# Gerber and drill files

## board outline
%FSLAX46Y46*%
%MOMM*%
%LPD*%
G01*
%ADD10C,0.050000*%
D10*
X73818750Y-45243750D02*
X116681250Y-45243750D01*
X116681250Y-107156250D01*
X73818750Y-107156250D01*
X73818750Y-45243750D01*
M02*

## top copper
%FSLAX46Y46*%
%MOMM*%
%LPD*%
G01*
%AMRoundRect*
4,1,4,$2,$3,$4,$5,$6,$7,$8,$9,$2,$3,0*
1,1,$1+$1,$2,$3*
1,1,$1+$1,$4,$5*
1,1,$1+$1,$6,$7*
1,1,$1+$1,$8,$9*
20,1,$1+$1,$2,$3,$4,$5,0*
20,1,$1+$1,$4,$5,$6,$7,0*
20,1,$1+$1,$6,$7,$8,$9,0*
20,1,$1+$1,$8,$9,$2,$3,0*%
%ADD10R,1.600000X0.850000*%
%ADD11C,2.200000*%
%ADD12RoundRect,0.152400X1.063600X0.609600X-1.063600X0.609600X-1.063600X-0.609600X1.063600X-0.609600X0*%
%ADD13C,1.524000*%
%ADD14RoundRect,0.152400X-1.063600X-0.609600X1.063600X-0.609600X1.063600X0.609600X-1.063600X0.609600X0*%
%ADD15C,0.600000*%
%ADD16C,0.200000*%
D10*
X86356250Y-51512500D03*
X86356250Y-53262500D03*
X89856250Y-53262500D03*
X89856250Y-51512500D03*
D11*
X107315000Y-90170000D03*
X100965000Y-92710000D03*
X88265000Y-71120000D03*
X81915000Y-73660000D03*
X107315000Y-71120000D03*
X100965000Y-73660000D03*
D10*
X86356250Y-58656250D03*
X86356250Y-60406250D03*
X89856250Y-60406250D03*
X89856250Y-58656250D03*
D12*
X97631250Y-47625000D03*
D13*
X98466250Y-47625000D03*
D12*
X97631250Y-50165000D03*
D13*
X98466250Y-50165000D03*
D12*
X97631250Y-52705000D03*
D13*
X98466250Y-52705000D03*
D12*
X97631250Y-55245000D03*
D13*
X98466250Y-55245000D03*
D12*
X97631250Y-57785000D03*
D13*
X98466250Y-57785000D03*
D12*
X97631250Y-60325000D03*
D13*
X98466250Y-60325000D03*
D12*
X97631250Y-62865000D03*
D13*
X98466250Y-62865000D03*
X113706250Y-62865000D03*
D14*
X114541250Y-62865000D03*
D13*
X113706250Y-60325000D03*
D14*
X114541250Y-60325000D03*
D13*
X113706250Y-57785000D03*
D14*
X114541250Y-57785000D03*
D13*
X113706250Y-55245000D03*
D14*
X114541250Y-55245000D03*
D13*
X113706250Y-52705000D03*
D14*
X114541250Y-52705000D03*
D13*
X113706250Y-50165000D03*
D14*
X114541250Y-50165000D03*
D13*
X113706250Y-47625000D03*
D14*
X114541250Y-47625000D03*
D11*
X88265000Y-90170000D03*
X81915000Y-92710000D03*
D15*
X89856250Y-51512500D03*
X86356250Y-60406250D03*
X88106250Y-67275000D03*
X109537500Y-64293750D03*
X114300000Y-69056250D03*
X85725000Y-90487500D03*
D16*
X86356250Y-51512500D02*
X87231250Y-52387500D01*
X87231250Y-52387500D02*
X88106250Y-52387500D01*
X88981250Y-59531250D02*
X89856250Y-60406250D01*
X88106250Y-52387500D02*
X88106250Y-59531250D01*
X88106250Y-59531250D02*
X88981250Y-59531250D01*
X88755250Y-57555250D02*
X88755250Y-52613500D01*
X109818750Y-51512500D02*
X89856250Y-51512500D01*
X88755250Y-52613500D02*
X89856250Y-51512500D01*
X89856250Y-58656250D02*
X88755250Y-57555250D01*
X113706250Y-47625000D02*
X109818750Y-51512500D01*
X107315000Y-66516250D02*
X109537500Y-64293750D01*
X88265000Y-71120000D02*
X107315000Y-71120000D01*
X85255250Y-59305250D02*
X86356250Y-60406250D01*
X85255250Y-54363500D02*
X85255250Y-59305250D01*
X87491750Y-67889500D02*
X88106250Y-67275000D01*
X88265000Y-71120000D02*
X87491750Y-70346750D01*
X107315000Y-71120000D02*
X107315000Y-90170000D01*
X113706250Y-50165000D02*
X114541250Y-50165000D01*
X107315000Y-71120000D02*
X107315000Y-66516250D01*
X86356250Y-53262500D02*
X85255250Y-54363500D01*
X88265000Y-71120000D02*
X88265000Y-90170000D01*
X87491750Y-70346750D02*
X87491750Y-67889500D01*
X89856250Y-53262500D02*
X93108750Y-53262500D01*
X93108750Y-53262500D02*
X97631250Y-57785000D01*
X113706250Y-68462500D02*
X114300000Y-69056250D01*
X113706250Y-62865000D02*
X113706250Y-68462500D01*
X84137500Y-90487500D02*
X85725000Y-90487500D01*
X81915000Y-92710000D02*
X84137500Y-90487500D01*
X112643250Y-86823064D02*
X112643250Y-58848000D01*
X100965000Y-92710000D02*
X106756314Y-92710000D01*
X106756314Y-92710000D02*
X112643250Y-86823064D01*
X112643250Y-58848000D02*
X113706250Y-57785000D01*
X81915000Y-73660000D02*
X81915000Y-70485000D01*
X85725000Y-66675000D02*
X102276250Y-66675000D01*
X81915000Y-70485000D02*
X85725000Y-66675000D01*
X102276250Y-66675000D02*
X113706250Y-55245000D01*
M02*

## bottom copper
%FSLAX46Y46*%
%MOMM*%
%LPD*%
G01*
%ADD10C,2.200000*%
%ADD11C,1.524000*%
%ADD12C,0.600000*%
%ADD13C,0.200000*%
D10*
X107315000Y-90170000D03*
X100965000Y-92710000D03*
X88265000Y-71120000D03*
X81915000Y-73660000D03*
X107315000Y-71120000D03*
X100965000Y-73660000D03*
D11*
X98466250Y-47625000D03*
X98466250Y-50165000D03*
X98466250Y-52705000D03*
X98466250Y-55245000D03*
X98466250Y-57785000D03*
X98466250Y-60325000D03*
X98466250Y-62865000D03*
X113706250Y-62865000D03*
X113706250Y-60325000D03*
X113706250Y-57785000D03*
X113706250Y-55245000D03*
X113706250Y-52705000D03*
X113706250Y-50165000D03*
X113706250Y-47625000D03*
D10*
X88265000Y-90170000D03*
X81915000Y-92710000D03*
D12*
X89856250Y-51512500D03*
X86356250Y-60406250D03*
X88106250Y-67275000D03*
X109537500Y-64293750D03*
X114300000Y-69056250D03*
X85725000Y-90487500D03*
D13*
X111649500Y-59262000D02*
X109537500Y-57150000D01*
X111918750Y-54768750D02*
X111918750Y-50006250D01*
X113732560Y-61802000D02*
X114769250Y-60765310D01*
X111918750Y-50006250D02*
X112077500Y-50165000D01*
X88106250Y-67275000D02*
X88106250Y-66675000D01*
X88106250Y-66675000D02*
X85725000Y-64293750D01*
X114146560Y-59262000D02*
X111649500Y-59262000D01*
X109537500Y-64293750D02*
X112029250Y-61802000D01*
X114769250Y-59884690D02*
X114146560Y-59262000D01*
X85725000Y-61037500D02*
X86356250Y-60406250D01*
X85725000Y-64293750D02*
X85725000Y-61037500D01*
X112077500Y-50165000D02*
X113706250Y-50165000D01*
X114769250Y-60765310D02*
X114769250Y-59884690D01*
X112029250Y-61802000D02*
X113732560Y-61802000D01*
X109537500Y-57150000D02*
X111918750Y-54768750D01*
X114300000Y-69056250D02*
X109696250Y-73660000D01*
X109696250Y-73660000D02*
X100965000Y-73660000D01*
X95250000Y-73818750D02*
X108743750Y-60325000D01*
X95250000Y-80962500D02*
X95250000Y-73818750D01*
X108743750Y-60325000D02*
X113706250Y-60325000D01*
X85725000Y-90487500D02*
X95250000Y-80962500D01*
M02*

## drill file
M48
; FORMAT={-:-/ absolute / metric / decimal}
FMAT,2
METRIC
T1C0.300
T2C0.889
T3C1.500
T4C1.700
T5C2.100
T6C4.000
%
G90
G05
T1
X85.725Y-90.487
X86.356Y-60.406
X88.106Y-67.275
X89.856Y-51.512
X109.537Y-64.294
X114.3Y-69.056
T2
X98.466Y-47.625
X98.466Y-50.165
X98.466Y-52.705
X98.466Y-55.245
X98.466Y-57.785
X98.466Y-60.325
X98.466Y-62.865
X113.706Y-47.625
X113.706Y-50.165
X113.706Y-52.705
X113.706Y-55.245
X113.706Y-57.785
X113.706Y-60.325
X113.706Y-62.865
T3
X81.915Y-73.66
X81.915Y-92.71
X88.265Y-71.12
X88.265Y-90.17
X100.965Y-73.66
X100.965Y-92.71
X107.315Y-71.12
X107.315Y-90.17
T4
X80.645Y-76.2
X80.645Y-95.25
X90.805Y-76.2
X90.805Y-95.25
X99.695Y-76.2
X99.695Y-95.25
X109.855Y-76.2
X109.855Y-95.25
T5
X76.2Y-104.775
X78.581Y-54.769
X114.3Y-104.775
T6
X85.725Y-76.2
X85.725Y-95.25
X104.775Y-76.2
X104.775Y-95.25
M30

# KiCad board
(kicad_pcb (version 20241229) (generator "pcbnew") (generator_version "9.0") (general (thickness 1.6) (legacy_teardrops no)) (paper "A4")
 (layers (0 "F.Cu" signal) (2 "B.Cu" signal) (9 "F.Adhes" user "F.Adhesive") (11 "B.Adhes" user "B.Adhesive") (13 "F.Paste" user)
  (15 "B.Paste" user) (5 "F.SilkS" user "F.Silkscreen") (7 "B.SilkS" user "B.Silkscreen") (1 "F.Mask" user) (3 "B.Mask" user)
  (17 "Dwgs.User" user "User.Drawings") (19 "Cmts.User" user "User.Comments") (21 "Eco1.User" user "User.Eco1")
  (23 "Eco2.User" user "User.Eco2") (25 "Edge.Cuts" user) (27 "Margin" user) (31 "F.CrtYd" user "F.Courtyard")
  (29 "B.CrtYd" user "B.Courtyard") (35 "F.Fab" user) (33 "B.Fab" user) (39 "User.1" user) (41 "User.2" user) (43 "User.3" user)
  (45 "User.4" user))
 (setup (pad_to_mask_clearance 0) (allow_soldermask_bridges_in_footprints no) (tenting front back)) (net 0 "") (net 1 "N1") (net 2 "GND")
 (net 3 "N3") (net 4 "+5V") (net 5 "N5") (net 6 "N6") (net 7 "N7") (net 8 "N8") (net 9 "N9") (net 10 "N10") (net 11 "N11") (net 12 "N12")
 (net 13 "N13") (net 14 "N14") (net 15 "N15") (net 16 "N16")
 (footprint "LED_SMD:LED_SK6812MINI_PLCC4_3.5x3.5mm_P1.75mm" (layer "F.Cu") (at 88.10625 52.3875)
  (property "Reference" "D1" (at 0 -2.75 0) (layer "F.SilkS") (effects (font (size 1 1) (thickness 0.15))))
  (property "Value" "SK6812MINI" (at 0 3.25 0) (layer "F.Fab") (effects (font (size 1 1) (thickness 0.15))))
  (pad "1" smd rect (at -1.75 -0.875) (size 1.6 0.85) (layers "F.Cu" "F.Mask" "F.Paste") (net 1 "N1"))
  (pad "2" smd rect (at -1.75 0.875) (size 1.6 0.85) (layers "F.Cu" "F.Mask" "F.Paste") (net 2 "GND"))
  (pad "3" smd rect (at 1.75 0.875) (size 1.6 0.85) (layers "F.Cu" "F.Mask" "F.Paste") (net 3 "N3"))
  (pad "4" smd rect (at 1.75 -0.875) (size 1.6 0.85) (layers "F.Cu" "F.Mask" "F.Paste") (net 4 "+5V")))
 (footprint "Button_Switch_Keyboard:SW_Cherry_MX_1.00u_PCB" (layer "F.Cu") (at 107.315 90.17)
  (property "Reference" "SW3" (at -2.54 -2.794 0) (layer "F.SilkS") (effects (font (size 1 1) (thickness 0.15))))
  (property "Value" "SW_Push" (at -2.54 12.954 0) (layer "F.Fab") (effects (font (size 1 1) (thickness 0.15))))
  (pad "" np_thru_hole circle (at -7.62 5.08) (size 1.7 1.7) (drill 1.7) (layers "*.Cu" "*.Mask"))
  (pad "" np_thru_hole circle (at -2.54 5.08) (size 4 4) (drill 4) (layers "*.Cu" "*.Mask"))
  (pad "" np_thru_hole circle (at 2.54 5.08) (size 1.7 1.7) (drill 1.7) (layers "*.Cu" "*.Mask"))
  (pad "1" thru_hole circle (at 0 0) (size 2.2 2.2) (drill 1.5) (layers "*.Cu" "*.Mask") (remove_unused_layers no) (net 2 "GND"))
  (pad "2" thru_hole circle (at -6.35 2.54) (size 2.2 2.2) (drill 1.5) (layers "*.Cu" "*.Mask") (remove_unused_layers no) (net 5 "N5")))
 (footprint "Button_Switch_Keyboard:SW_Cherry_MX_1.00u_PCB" (layer "F.Cu") (at 88.265 71.12)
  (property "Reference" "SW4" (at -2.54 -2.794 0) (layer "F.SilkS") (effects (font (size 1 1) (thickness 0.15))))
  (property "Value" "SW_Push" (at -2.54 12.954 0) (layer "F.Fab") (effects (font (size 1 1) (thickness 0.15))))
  (pad "" np_thru_hole circle (at -7.62 5.08) (size 1.7 1.7) (drill 1.7) (layers "*.Cu" "*.Mask"))
  (pad "" np_thru_hole circle (at -2.54 5.08) (size 4 4) (drill 4) (layers "*.Cu" "*.Mask"))
  (pad "" np_thru_hole circle (at 2.54 5.08) (size 1.7 1.7) (drill 1.7) (layers "*.Cu" "*.Mask"))
  (pad "1" thru_hole circle (at 0 0) (size 2.2 2.2) (drill 1.5) (layers "*.Cu" "*.Mask") (remove_unused_layers no) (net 2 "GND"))
  (pad "2" thru_hole circle (at -6.35 2.54) (size 2.2 2.2) (drill 1.5) (layers "*.Cu" "*.Mask") (remove_unused_layers no) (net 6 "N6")))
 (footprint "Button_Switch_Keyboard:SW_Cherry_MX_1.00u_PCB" (layer "F.Cu") (at 107.315 71.12)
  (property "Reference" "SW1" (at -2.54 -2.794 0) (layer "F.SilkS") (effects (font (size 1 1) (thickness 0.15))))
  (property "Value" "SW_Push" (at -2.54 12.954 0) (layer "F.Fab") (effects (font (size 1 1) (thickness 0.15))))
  (pad "" np_thru_hole circle (at -7.62 5.08) (size 1.7 1.7) (drill 1.7) (layers "*.Cu" "*.Mask"))
  (pad "" np_thru_hole circle (at -2.54 5.08) (size 4 4) (drill 4) (layers "*.Cu" "*.Mask"))
  (pad "" np_thru_hole circle (at 2.54 5.08) (size 1.7 1.7) (drill 1.7) (layers "*.Cu" "*.Mask"))
  (pad "1" thru_hole circle (at 0 0) (size 2.2 2.2) (drill 1.5) (layers "*.Cu" "*.Mask") (remove_unused_layers no) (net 2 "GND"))
  (pad "2" thru_hole circle (at -6.35 2.54) (size 2.2 2.2) (drill 1.5) (layers "*.Cu" "*.Mask") (remove_unused_layers no) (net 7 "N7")))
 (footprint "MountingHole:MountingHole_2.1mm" (layer "F.Cu") (at 76.2 104.775)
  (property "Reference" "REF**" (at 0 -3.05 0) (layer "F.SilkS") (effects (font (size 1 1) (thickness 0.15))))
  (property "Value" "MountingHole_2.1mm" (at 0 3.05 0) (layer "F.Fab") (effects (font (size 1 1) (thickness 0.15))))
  (pad "" np_thru_hole circle (at 0 0) (size 2.1 2.1) (drill 2.1) (layers "*.Cu" "*.Mask")))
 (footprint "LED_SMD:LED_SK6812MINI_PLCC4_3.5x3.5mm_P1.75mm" (layer "F.Cu") (at 88.10625 59.53125)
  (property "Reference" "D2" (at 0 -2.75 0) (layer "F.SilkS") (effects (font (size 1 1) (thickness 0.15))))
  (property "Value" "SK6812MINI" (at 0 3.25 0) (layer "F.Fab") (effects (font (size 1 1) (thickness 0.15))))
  (pad "1" smd rect (at -1.75 -0.875) (size 1.6 0.85) (layers "F.Cu" "F.Mask" "F.Paste") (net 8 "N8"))
  (pad "2" smd rect (at -1.75 0.875) (size 1.6 0.85) (layers "F.Cu" "F.Mask" "F.Paste") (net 2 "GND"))
  (pad "3" smd rect (at 1.75 0.875) (size 1.6 0.85) (layers "F.Cu" "F.Mask" "F.Paste") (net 1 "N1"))
  (pad "4" smd rect (at 1.75 -0.875) (size 1.6 0.85) (layers "F.Cu" "F.Mask" "F.Paste") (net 4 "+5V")))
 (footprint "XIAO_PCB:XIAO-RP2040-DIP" (layer "F.Cu") (at 106.08625 55.245)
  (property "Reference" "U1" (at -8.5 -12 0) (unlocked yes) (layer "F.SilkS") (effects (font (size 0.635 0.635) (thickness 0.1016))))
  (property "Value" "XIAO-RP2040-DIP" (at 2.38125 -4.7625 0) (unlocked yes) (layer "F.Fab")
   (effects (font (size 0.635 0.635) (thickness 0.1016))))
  (pad "1" smd roundrect (at -8.455 -7.62 180) (size 2.432 1.524) (layers "F.Cu" "F.Mask") (roundrect_rratio 0.1) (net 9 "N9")
   (thermal_bridge_angle 45))
  (pad "1" thru_hole circle (at -7.62 -7.62 180) (size 1.524 1.524) (drill 0.889) (layers "*.Cu" "*.Mask") (remove_unused_layers no)
   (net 9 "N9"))
  (pad "2" smd roundrect (at -8.455 -5.08 180) (size 2.432 1.524) (layers "F.Cu" "F.Mask") (roundrect_rratio 0.1) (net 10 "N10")
   (thermal_bridge_angle 45))
  (pad "2" thru_hole circle (at -7.62 -5.08 180) (size 1.524 1.524) (drill 0.889) (layers "*.Cu" "*.Mask") (remove_unused_layers no)
   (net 10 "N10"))
  (pad "3" smd roundrect (at -8.455 -2.54 180) (size 2.432 1.524) (layers "F.Cu" "F.Mask") (roundrect_rratio 0.1) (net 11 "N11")
   (thermal_bridge_angle 45))
  (pad "3" thru_hole circle (at -7.62 -2.54 180) (size 1.524 1.524) (drill 0.889) (layers "*.Cu" "*.Mask") (remove_unused_layers no)
   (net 11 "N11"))
  (pad "4" smd roundrect (at -8.455 0 180) (size 2.432 1.524) (layers "F.Cu" "F.Mask") (roundrect_rratio 0.1) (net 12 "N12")
   (thermal_bridge_angle 45))
  (pad "4" thru_hole circle (at -7.62 0 180) (size 1.524 1.524) (drill 0.889) (layers "*.Cu" "*.Mask") (remove_unused_layers no)
   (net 12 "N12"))
  (pad "5" smd roundrect (at -8.455 2.54 180) (size 2.432 1.524) (layers "F.Cu" "F.Mask") (roundrect_rratio 0.1) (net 3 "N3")
   (thermal_bridge_angle 45))
  (pad "5" thru_hole circle (at -7.62 2.54 180) (size 1.524 1.524) (drill 0.889) (layers "*.Cu" "*.Mask") (remove_unused_layers no)
   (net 3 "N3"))
  (pad "6" smd roundrect (at -8.455 5.08 180) (size 2.432 1.524) (layers "F.Cu" "F.Mask") (roundrect_rratio 0.1) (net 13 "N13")
   (thermal_bridge_angle 45))
  (pad "6" thru_hole circle (at -7.62 5.08 180) (size 1.524 1.524) (drill 0.889) (layers "*.Cu" "*.Mask") (remove_unused_layers no)
   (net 13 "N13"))
  (pad "7" smd roundrect (at -8.455 7.62 180) (size 2.432 1.524) (layers "F.Cu" "F.Mask") (roundrect_rratio 0.1) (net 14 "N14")
   (thermal_bridge_angle 45))
  (pad "7" thru_hole circle (at -7.62 7.62 180) (size 1.524 1.524) (drill 0.889) (layers "*.Cu" "*.Mask") (remove_unused_layers no)
   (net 14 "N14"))
  (pad "8" thru_hole circle (at 7.62 7.62) (size 1.524 1.524) (drill 0.889) (layers "*.Cu" "*.Mask") (remove_unused_layers no) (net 7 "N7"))
  (pad "8" smd roundrect (at 8.455 7.62) (size 2.432 1.524) (layers "F.Cu" "F.Mask") (roundrect_rratio 0.1) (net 7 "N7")
   (thermal_bridge_angle 45))
  (pad "9" thru_hole circle (at 7.62 5.08) (size 1.524 1.524) (drill 0.889) (layers "*.Cu" "*.Mask") (remove_unused_layers no)
   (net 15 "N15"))
  (pad "9" smd roundrect (at 8.455 5.08) (size 2.432 1.524) (layers "F.Cu" "F.Mask") (roundrect_rratio 0.1) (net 15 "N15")
   (thermal_bridge_angle 45))
  (pad "10" thru_hole circle (at 7.62 2.54) (size 1.524 1.524) (drill 0.889) (layers "*.Cu" "*.Mask") (remove_unused_layers no) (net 5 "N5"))
  (pad "10" smd roundrect (at 8.455 2.54) (size 2.432 1.524) (layers "F.Cu" "F.Mask") (roundrect_rratio 0.1) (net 5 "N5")
   (thermal_bridge_angle 45))
  (pad "11" thru_hole circle (at 7.62 0) (size 1.524 1.524) (drill 0.889) (layers "*.Cu" "*.Mask") (remove_unused_layers no) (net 6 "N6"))
  (pad "11" smd roundrect (at 8.455 0) (size 2.432 1.524) (layers "F.Cu" "F.Mask") (roundrect_rratio 0.1) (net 6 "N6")
   (thermal_bridge_angle 45))
  (pad "12" thru_hole circle (at 7.62 -2.54) (size 1.524 1.524) (drill 0.889) (layers "*.Cu" "*.Mask") (remove_unused_layers no)
   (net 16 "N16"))
  (pad "12" smd roundrect (at 8.455 -2.54) (size 2.432 1.524) (layers "F.Cu" "F.Mask") (roundrect_rratio 0.1) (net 16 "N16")
   (thermal_bridge_angle 45))
  (pad "13" thru_hole circle (at 7.62 -5.08) (size 1.524 1.524) (drill 0.889) (layers "*.Cu" "*.Mask") (remove_unused_layers no)
   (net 2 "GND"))
  (pad "13" smd roundrect (at 8.455 -5.08) (size 2.432 1.524) (layers "F.Cu" "F.Mask") (roundrect_rratio 0.1) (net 2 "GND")
   (thermal_bridge_angle 45))
  (pad "14" thru_hole circle (at 7.62 -7.62) (size 1.524 1.524) (drill 0.889) (layers "*.Cu" "*.Mask") (remove_unused_layers no)
   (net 4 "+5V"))
  (pad "14" smd roundrect (at 8.455 -7.62) (size 2.432 1.524) (layers "F.Cu" "F.Mask") (roundrect_rratio 0.1) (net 4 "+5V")
   (thermal_bridge_angle 45)))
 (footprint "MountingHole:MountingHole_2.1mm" (layer "F.Cu") (at 78.58125 54.76875)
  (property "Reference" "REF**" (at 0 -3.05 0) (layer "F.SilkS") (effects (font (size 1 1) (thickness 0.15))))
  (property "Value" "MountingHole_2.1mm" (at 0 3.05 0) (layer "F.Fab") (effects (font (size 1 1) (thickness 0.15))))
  (pad "" np_thru_hole circle (at 0 0) (size 2.1 2.1) (drill 2.1) (layers "*.Cu" "*.Mask")))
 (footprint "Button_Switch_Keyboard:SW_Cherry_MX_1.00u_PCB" (layer "F.Cu") (at 88.265 90.17)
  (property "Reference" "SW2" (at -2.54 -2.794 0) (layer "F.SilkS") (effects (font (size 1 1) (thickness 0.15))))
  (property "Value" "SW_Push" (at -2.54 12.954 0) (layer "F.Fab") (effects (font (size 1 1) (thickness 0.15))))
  (pad "" np_thru_hole circle (at -7.62 5.08) (size 1.7 1.7) (drill 1.7) (layers "*.Cu" "*.Mask"))
  (pad "" np_thru_hole circle (at -2.54 5.08) (size 4 4) (drill 4) (layers "*.Cu" "*.Mask"))
  (pad "" np_thru_hole circle (at 2.54 5.08) (size 1.7 1.7) (drill 1.7) (layers "*.Cu" "*.Mask"))
  (pad "1" thru_hole circle (at 0 0) (size 2.2 2.2) (drill 1.5) (layers "*.Cu" "*.Mask") (remove_unused_layers no) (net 2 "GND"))
  (pad "2" thru_hole circle (at -6.35 2.54) (size 2.2 2.2) (drill 1.5) (layers "*.Cu" "*.Mask") (remove_unused_layers no) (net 15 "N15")))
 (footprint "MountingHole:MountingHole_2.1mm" (layer "F.Cu") (at 114.3 104.775)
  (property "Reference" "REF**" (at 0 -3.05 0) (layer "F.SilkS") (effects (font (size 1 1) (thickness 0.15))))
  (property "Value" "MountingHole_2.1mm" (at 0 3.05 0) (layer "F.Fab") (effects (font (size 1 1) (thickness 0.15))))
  (pad "" np_thru_hole circle (at 0 0) (size 2.1 2.1) (drill 2.1) (layers "*.Cu" "*.Mask")))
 (gr_rect (start 73.81875 45.24375) (end 116.68125 107.15625) (stroke (width 0.05) (type default)) (fill no) (layer "Edge.Cuts"))
 (segment (start 86.35625 51.5125) (end 87.23125 52.3875) (width 0.2) (layer "F.Cu") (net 1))
 (segment (start 87.23125 52.3875) (end 88.10625 52.3875) (width 0.2) (layer "F.Cu") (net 1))
 (segment (start 88.98125 59.53125) (end 89.85625 60.40625) (width 0.2) (layer "F.Cu") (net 1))
 (segment (start 88.10625 52.3875) (end 88.10625 59.53125) (width 0.2) (layer "F.Cu") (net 1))
 (segment (start 88.10625 59.53125) (end 88.98125 59.53125) (width 0.2) (layer "F.Cu") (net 1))
 (segment (start 88.75525 57.55525) (end 88.75525 52.6135) (width 0.2) (layer "F.Cu") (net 4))
 (segment (start 109.81875 51.5125) (end 89.85625 51.5125) (width 0.2) (layer "F.Cu") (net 4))
 (segment (start 88.75525 52.6135) (end 89.85625 51.5125) (width 0.2) (layer "F.Cu") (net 4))
 (segment (start 89.85625 58.65625) (end 88.75525 57.55525) (width 0.2) (layer "F.Cu") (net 4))
 (segment (start 113.70625 47.625) (end 109.81875 51.5125) (width 0.2) (layer "F.Cu") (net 4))
 (via (at 89.85625 51.5125) (size 0.6) (drill 0.3) (layers "F.Cu" "B.Cu") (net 4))
 (segment (start 107.315 66.51625) (end 109.5375 64.29375) (width 0.2) (layer "F.Cu") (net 2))
 (segment (start 88.265 71.12) (end 107.315 71.12) (width 0.2) (layer "F.Cu") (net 2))
 (segment (start 85.25525 59.30525) (end 86.35625 60.40625) (width 0.2) (layer "F.Cu") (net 2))
 (segment (start 85.25525 54.3635) (end 85.25525 59.30525) (width 0.2) (layer "F.Cu") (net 2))
 (segment (start 87.49175 67.8895) (end 88.10625 67.275) (width 0.2) (layer "F.Cu") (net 2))
 (segment (start 88.265 71.12) (end 87.49175 70.34675) (width 0.2) (layer "F.Cu") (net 2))
 (segment (start 107.315 71.12) (end 107.315 90.17) (width 0.2) (layer "F.Cu") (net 2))
 (segment (start 113.70625 50.165) (end 114.54125 50.165) (width 0.2) (layer "F.Cu") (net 2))
 (segment (start 107.315 71.12) (end 107.315 66.51625) (width 0.2) (layer "F.Cu") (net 2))
 (segment (start 86.35625 53.2625) (end 85.25525 54.3635) (width 0.2) (layer "F.Cu") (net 2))
 (segment (start 88.265 71.12) (end 88.265 90.17) (width 0.2) (layer "F.Cu") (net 2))
 (segment (start 87.49175 70.34675) (end 87.49175 67.8895) (width 0.2) (layer "F.Cu") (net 2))
 (via (at 86.35625 60.40625) (size 0.6) (drill 0.3) (layers "F.Cu" "B.Cu") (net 2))
 (via (at 88.10625 67.275) (size 0.6) (drill 0.3) (layers "F.Cu" "B.Cu") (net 2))
 (via (at 109.5375 64.29375) (size 0.6) (drill 0.3) (layers "F.Cu" "B.Cu") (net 2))
 (segment (start 111.6495 59.262) (end 109.5375 57.15) (width 0.2) (layer "B.Cu") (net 2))
 (segment (start 111.91875 54.76875) (end 111.91875 50.00625) (width 0.2) (layer "B.Cu") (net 2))
 (segment (start 113.73256 61.802) (end 114.76925 60.76531) (width 0.2) (layer "B.Cu") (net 2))
 (segment (start 111.91875 50.00625) (end 112.0775 50.165) (width 0.2) (layer "B.Cu") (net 2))
 (segment (start 88.10625 67.275) (end 88.10625 66.675) (width 0.2) (layer "B.Cu") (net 2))
 (segment (start 88.10625 66.675) (end 85.725 64.29375) (width 0.2) (layer "B.Cu") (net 2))
 (segment (start 114.14656 59.262) (end 111.6495 59.262) (width 0.2) (layer "B.Cu") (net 2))
 (segment (start 109.5375 64.29375) (end 112.02925 61.802) (width 0.2) (layer "B.Cu") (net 2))
 (segment (start 114.76925 59.88469) (end 114.14656 59.262) (width 0.2) (layer "B.Cu") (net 2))
 (segment (start 85.725 61.0375) (end 86.35625 60.40625) (width 0.2) (layer "B.Cu") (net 2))
 (segment (start 85.725 64.29375) (end 85.725 61.0375) (width 0.2) (layer "B.Cu") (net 2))
 (segment (start 112.0775 50.165) (end 113.70625 50.165) (width 0.2) (layer "B.Cu") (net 2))
 (segment (start 114.76925 60.76531) (end 114.76925 59.88469) (width 0.2) (layer "B.Cu") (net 2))
 (segment (start 112.02925 61.802) (end 113.73256 61.802) (width 0.2) (layer "B.Cu") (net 2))
 (segment (start 109.5375 57.15) (end 111.91875 54.76875) (width 0.2) (layer "B.Cu") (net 2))
 (segment (start 89.85625 53.2625) (end 93.10875 53.2625) (width 0.2) (layer "F.Cu") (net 3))
 (segment (start 93.10875 53.2625) (end 97.63125 57.785) (width 0.2) (layer "F.Cu") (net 3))
 (segment (start 113.70625 68.4625) (end 114.3 69.05625) (width 0.2) (layer "F.Cu") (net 7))
 (segment (start 113.70625 62.865) (end 113.70625 68.4625) (width 0.2) (layer "F.Cu") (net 7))
 (via (at 114.3 69.05625) (size 0.6) (drill 0.3) (layers "F.Cu" "B.Cu") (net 7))
 (segment (start 114.3 69.05625) (end 109.69625 73.66) (width 0.2) (layer "B.Cu") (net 7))
 (segment (start 109.69625 73.66) (end 100.965 73.66) (width 0.2) (layer "B.Cu") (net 7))
 (segment (start 84.1375 90.4875) (end 85.725 90.4875) (width 0.2) (layer "F.Cu") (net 15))
 (segment (start 81.915 92.71) (end 84.1375 90.4875) (width 0.2) (layer "F.Cu") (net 15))
 (via (at 85.725 90.4875) (size 0.6) (drill 0.3) (layers "F.Cu" "B.Cu") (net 15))
 (segment (start 95.25 73.81875) (end 108.74375 60.325) (width 0.2) (layer "B.Cu") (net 15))
 (segment (start 95.25 80.9625) (end 95.25 73.81875) (width 0.2) (layer "B.Cu") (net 15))
 (segment (start 108.74375 60.325) (end 113.70625 60.325) (width 0.2) (layer "B.Cu") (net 15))
 (segment (start 85.725 90.4875) (end 95.25 80.9625) (width 0.2) (layer "B.Cu") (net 15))
 (segment (start 112.64325 86.823064) (end 112.64325 58.848) (width 0.2) (layer "F.Cu") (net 5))
 (segment (start 100.965 92.71) (end 106.756314 92.71) (width 0.2) (layer "F.Cu") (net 5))
 (segment (start 106.756314 92.71) (end 112.64325 86.823064) (width 0.2) (layer "F.Cu") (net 5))
 (segment (start 112.64325 58.848) (end 113.70625 57.785) (width 0.2) (layer "F.Cu") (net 5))
 (segment (start 81.915 73.66) (end 81.915 70.485) (width 0.2) (layer "F.Cu") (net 6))
 (segment (start 85.725 66.675) (end 102.27625 66.675) (width 0.2) (layer "F.Cu") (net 6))
 (segment (start 81.915 70.485) (end 85.725 66.675) (width 0.2) (layer "F.Cu") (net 6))
 (segment (start 102.27625 66.675) (end 113.70625 55.245) (width 0.2) (layer "F.Cu") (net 6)))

